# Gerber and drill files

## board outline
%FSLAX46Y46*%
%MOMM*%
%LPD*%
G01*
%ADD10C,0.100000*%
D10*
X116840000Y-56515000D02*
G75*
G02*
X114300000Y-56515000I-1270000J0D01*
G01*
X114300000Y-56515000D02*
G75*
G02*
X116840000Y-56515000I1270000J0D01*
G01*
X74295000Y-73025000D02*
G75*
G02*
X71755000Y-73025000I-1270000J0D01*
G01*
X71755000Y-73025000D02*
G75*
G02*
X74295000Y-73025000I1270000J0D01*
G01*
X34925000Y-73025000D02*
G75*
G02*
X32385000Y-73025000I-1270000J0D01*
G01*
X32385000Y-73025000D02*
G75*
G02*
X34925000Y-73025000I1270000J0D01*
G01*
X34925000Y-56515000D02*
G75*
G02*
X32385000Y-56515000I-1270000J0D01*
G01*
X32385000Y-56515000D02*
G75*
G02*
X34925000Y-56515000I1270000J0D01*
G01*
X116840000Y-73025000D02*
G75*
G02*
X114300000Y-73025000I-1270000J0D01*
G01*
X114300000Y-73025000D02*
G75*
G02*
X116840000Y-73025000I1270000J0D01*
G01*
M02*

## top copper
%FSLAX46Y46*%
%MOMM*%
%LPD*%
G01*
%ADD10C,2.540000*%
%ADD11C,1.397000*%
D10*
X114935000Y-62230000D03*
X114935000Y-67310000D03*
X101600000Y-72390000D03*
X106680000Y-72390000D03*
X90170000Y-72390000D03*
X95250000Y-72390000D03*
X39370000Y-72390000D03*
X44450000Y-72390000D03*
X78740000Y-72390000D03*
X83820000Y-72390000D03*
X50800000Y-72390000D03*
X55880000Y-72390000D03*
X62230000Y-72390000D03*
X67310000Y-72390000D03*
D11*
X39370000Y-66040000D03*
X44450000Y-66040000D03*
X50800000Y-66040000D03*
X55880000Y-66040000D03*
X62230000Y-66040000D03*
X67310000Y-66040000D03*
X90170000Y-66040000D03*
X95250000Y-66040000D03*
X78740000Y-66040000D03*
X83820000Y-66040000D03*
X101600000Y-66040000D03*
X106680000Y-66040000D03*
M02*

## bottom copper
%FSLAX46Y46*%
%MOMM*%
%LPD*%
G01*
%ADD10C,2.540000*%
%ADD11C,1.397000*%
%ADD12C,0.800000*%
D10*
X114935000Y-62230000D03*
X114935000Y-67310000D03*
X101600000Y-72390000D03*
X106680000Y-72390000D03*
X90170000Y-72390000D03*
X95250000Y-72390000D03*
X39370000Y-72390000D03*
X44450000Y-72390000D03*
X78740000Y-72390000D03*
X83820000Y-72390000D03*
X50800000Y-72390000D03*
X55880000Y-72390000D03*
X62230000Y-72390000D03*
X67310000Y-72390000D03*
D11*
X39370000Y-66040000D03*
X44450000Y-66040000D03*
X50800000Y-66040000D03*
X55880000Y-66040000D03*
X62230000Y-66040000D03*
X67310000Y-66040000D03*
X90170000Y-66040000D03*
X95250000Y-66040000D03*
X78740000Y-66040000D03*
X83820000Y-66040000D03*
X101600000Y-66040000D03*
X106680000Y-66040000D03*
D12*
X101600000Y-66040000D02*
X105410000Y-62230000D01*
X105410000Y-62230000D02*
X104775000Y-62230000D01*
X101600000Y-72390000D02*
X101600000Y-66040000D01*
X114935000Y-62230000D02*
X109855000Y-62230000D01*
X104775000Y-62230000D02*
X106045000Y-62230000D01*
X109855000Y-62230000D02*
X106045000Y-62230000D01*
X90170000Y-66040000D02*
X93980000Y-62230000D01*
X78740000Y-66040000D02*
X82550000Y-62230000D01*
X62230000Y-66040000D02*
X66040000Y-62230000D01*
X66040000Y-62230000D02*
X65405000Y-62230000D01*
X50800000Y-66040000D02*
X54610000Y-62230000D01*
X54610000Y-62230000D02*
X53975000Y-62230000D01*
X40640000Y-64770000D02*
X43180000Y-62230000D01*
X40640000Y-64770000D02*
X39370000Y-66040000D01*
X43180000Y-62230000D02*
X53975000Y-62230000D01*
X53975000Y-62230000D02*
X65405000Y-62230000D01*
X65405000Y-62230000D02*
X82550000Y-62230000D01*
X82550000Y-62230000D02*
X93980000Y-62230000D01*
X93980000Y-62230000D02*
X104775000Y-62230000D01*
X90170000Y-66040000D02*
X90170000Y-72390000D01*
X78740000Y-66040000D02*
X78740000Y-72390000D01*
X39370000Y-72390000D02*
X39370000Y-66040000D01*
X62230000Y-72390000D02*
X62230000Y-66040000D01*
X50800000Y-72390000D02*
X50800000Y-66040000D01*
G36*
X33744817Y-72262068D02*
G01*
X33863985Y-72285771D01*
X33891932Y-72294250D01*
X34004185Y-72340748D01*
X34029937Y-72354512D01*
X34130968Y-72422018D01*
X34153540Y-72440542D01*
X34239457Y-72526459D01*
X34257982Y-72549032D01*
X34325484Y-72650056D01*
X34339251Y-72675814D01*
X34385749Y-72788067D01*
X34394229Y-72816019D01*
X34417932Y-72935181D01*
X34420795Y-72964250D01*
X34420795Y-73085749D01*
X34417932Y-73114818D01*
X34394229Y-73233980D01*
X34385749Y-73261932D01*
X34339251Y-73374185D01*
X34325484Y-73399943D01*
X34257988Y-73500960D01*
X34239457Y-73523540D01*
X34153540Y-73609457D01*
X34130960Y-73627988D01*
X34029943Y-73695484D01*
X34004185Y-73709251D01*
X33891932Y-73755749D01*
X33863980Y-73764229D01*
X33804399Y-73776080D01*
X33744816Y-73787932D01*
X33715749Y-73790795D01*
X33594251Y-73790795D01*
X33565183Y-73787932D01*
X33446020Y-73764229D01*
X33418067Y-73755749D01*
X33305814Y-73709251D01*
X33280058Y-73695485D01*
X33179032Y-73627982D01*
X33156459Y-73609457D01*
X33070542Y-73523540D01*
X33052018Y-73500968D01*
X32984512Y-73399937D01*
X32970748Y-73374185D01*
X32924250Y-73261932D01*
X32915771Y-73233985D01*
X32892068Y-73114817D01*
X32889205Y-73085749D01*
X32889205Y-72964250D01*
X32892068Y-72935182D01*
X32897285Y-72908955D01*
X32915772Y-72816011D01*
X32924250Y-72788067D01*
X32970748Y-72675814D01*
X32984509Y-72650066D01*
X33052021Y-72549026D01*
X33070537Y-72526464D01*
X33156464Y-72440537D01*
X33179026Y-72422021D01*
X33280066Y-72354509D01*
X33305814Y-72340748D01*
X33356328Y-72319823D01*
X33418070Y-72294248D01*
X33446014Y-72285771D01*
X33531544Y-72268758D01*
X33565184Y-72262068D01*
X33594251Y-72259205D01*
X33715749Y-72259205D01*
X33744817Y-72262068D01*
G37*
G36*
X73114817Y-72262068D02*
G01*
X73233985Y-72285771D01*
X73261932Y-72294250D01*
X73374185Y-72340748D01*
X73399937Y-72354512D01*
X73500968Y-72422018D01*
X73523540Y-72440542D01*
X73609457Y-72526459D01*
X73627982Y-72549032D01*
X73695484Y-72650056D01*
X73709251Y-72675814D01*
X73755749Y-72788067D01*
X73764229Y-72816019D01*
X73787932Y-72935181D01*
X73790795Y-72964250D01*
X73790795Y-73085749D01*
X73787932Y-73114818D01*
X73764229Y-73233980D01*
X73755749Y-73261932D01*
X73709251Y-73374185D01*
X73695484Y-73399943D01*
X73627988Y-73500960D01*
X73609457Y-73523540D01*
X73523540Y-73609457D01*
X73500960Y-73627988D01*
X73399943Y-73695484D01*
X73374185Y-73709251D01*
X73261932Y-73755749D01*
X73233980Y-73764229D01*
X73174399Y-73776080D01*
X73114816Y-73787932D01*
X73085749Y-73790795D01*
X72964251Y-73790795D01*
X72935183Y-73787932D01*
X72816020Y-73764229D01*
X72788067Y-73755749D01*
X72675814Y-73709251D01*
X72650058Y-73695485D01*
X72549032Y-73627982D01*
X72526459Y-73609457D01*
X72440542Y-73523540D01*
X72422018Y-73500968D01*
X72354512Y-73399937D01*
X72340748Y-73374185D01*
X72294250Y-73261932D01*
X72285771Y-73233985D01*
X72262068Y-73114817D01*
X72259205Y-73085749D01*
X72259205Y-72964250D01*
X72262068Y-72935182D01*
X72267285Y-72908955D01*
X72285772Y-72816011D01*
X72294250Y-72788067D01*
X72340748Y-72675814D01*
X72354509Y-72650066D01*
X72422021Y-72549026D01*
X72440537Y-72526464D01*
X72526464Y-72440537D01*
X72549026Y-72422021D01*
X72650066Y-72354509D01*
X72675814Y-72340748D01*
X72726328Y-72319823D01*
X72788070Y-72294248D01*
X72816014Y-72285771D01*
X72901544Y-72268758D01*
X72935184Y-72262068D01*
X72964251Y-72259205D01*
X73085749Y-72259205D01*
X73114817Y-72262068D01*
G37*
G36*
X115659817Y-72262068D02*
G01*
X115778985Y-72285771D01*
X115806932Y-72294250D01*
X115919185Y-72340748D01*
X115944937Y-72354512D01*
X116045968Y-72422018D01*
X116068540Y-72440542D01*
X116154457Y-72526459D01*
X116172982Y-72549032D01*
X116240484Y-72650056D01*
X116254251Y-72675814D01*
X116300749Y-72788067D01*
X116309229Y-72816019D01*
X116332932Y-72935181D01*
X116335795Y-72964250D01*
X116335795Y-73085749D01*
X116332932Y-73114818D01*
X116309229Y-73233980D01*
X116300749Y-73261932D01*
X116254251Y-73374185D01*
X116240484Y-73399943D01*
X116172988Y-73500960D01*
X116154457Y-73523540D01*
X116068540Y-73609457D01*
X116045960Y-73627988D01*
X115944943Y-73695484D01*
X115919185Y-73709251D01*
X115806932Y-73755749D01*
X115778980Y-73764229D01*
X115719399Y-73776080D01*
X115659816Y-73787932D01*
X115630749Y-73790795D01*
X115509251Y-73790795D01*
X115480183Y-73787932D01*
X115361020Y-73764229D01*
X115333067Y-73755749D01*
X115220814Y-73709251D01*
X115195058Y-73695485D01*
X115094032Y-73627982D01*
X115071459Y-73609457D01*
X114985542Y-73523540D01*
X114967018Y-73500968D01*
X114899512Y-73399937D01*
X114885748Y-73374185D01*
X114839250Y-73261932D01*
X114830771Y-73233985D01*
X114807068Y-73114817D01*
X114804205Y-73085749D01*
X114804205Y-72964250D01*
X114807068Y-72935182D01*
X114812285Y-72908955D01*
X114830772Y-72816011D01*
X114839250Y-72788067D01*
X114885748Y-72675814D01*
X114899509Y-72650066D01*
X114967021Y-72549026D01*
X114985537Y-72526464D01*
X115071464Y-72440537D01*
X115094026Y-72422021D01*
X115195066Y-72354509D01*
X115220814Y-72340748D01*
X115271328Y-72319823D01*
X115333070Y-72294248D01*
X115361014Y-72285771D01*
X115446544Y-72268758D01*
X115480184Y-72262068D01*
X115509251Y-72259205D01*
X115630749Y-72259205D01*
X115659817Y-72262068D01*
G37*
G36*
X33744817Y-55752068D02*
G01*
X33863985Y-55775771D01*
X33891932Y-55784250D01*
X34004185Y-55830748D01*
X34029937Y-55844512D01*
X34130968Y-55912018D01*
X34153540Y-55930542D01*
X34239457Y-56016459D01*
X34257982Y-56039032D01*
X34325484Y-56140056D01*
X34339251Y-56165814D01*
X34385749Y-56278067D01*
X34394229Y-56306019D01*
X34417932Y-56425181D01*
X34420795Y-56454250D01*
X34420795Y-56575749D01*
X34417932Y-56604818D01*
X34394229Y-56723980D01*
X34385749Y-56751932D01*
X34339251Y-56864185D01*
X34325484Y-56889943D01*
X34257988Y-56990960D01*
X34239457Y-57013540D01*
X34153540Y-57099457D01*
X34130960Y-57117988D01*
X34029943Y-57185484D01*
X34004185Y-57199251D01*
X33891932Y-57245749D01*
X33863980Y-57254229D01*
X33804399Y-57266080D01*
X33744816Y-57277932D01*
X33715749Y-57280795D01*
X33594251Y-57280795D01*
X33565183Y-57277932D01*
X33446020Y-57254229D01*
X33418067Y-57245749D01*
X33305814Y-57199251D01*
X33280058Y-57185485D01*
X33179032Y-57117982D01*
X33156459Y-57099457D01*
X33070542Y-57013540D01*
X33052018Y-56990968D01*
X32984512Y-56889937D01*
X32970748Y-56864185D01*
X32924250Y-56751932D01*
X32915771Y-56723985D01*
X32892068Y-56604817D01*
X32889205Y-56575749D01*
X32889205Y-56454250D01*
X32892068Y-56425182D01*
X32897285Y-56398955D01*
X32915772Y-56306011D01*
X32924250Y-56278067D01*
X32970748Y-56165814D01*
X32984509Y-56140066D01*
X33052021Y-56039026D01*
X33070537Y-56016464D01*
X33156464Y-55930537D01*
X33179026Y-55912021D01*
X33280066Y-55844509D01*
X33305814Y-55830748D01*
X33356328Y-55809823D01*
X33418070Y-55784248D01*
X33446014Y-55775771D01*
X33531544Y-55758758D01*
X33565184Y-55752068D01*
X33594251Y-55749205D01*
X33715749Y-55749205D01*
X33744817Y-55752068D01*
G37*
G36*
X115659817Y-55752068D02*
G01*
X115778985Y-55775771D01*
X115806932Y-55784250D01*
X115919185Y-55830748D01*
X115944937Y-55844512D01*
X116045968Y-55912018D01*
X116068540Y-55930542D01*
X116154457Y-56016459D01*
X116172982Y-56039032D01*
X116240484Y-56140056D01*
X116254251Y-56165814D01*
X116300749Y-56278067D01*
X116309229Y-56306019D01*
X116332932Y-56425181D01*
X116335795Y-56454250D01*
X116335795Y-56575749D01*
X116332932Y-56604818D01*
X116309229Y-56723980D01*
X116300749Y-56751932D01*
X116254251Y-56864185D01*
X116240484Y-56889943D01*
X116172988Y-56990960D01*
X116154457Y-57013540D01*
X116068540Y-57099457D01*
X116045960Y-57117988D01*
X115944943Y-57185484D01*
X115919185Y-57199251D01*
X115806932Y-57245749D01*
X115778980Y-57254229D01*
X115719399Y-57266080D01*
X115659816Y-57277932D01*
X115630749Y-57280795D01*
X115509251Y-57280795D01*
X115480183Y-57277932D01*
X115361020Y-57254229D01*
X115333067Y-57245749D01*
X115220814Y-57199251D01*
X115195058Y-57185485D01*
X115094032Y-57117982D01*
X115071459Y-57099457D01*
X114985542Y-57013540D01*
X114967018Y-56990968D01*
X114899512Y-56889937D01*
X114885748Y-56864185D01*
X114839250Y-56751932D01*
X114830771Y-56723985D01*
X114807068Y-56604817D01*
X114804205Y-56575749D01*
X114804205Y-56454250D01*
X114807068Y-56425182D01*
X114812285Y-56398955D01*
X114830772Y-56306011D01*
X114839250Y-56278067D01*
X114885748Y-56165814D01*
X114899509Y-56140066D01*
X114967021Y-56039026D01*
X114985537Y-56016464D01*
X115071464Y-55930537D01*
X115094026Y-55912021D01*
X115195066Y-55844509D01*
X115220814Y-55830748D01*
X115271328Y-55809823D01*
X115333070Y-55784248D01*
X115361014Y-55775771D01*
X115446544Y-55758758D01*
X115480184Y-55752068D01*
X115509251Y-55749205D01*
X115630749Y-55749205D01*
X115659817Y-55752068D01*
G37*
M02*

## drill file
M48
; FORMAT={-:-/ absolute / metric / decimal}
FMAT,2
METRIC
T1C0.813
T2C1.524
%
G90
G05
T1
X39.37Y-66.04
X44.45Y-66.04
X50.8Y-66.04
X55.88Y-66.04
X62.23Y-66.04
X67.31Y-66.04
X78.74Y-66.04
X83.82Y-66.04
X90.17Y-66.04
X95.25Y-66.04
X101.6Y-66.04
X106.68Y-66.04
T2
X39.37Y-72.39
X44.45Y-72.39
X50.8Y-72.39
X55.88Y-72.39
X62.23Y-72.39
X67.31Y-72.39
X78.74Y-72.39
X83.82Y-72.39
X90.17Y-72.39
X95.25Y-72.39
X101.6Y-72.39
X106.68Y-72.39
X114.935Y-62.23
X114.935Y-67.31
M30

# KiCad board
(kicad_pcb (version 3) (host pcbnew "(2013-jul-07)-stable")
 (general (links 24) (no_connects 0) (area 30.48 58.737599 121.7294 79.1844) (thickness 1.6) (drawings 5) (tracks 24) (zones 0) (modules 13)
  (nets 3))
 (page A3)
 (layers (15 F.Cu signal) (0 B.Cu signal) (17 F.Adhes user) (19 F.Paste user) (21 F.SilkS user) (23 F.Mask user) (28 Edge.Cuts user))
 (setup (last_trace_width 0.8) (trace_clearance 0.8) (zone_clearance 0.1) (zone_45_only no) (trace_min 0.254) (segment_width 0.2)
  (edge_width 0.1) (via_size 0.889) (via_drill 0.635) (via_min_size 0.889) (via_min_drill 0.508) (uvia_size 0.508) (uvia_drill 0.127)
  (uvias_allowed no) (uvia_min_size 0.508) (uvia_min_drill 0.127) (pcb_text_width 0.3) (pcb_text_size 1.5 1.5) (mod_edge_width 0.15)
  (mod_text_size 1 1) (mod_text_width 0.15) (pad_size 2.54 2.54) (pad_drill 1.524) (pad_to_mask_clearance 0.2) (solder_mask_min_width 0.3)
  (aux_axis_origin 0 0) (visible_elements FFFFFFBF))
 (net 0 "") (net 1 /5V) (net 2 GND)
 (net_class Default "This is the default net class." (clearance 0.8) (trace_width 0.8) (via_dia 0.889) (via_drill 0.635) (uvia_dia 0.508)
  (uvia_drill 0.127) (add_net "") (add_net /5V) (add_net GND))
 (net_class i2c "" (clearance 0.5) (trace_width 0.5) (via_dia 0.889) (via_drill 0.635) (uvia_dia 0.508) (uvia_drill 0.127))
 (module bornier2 (layer F.Cu) (at 114.935 64.77 270)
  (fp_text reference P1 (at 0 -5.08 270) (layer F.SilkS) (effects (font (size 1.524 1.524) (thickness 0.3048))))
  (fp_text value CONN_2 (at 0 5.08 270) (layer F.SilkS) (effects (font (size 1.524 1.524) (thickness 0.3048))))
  (pad 1 thru_hole circle (at -2.54 0 270) (size 2.54 2.54) (drill 1.524) (layers *.Cu *.Mask F.SilkS) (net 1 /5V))
  (pad 2 thru_hole circle (at 2.54 0 270) (size 2.54 2.54) (drill 1.524) (layers *.Cu *.Mask F.SilkS) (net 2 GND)))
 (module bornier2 (layer F.Cu) (at 104.14 72.39)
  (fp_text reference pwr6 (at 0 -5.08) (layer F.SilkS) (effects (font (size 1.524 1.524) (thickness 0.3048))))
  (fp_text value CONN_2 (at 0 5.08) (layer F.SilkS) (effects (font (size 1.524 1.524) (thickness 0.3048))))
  (pad 1 thru_hole circle (at -2.54 0) (size 2.54 2.54) (drill 1.524) (layers *.Cu *.Mask F.SilkS) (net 1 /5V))
  (pad 2 thru_hole circle (at 2.54 0) (size 2.54 2.54) (drill 1.524) (layers *.Cu *.Mask F.SilkS) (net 2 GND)))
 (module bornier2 (layer F.Cu) (at 92.71 72.39)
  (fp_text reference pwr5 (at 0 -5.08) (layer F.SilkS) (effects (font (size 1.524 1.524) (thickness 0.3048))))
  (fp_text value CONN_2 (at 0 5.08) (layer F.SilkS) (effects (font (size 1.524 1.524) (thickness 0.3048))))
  (pad 1 thru_hole circle (at -2.54 0) (size 2.54 2.54) (drill 1.524) (layers *.Cu *.Mask F.SilkS) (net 1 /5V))
  (pad 2 thru_hole circle (at 2.54 0) (size 2.54 2.54) (drill 1.524) (layers *.Cu *.Mask F.SilkS) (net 2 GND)))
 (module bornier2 (layer F.Cu) (at 41.91 72.39)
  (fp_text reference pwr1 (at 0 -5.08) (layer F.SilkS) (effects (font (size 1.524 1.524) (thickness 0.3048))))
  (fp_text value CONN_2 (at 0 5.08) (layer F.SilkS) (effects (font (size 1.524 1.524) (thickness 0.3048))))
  (pad 1 thru_hole circle (at -2.54 0) (size 2.54 2.54) (drill 1.524) (layers *.Cu *.Mask F.SilkS) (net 1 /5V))
  (pad 2 thru_hole circle (at 2.54 0) (size 2.54 2.54) (drill 1.524) (layers *.Cu *.Mask F.SilkS) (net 2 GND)))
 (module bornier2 (layer F.Cu) (at 81.28 72.39)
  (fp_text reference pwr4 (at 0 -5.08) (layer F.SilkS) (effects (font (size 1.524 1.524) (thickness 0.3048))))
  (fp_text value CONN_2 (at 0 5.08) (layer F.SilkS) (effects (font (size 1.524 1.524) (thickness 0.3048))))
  (pad 1 thru_hole circle (at -2.54 0) (size 2.54 2.54) (drill 1.524) (layers *.Cu *.Mask F.SilkS) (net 1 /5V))
  (pad 2 thru_hole circle (at 2.54 0) (size 2.54 2.54) (drill 1.524) (layers *.Cu *.Mask F.SilkS) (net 2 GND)))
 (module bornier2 (layer F.Cu) (at 53.34 72.39)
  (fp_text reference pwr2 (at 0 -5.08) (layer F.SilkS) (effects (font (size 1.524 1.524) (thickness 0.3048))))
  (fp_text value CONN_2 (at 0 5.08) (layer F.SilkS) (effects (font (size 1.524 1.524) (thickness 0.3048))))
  (pad 1 thru_hole circle (at -2.54 0) (size 2.54 2.54) (drill 1.524) (layers *.Cu *.Mask F.SilkS) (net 1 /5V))
  (pad 2 thru_hole circle (at 2.54 0) (size 2.54 2.54) (drill 1.524) (layers *.Cu *.Mask F.SilkS) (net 2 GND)))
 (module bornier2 (layer F.Cu) (at 64.77 72.39)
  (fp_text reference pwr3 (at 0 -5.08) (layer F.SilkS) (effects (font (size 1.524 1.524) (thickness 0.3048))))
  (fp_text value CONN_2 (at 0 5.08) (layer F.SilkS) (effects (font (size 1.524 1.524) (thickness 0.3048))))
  (pad 1 thru_hole circle (at -2.54 0) (size 2.54 2.54) (drill 1.524) (layers *.Cu *.Mask F.SilkS) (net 1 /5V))
  (pad 2 thru_hole circle (at 2.54 0) (size 2.54 2.54) (drill 1.524) (layers *.Cu *.Mask F.SilkS) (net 2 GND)))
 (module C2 (layer F.Cu) (at 41.91 66.04)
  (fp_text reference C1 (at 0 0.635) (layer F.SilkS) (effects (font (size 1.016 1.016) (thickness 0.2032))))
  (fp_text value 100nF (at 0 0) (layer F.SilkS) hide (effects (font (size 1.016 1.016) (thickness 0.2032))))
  (pad 1 thru_hole circle (at -2.54 0) (size 1.397 1.397) (drill 0.8128) (layers *.Cu *.Mask F.SilkS) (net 1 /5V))
  (pad 2 thru_hole circle (at 2.54 0) (size 1.397 1.397) (drill 0.8128) (layers *.Cu *.Mask F.SilkS) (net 2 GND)))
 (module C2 (layer F.Cu) (at 53.34 66.04)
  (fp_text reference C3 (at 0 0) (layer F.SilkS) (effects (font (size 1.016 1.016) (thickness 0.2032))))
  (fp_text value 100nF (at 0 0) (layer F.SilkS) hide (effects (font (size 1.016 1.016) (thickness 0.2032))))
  (pad 1 thru_hole circle (at -2.54 0) (size 1.397 1.397) (drill 0.8128) (layers *.Cu *.Mask F.SilkS) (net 1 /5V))
  (pad 2 thru_hole circle (at 2.54 0) (size 1.397 1.397) (drill 0.8128) (layers *.Cu *.Mask F.SilkS) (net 2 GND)))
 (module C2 (layer F.Cu) (at 64.77 66.04)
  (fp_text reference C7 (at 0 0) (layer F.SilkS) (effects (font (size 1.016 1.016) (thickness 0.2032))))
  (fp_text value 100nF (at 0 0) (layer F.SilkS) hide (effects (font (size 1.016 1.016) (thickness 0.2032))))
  (pad 1 thru_hole circle (at -2.54 0) (size 1.397 1.397) (drill 0.8128) (layers *.Cu *.Mask F.SilkS) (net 1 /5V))
  (pad 2 thru_hole circle (at 2.54 0) (size 1.397 1.397) (drill 0.8128) (layers *.Cu *.Mask F.SilkS) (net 2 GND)))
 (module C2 (layer F.Cu) (at 92.71 66.04)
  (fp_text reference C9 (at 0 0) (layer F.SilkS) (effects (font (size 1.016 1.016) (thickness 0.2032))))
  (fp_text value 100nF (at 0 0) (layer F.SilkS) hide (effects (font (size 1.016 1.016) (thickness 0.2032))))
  (pad 1 thru_hole circle (at -2.54 0) (size 1.397 1.397) (drill 0.8128) (layers *.Cu *.Mask F.SilkS) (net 1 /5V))
  (pad 2 thru_hole circle (at 2.54 0) (size 1.397 1.397) (drill 0.8128) (layers *.Cu *.Mask F.SilkS) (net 2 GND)))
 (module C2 (layer F.Cu) (at 81.28 66.04)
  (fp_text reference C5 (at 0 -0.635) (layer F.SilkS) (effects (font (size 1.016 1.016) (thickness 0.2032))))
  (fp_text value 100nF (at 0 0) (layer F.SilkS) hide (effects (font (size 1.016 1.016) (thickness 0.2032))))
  (pad 1 thru_hole circle (at -2.54 0) (size 1.397 1.397) (drill 0.8128) (layers *.Cu *.Mask F.SilkS) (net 1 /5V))
  (pad 2 thru_hole circle (at 2.54 0) (size 1.397 1.397) (drill 0.8128) (layers *.Cu *.Mask F.SilkS) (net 2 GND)))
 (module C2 (layer F.Cu) (at 104.14 66.04)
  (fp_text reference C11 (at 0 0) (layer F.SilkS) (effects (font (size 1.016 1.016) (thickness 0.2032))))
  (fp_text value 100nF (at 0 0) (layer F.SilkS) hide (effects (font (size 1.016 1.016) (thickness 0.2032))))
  (pad 1 thru_hole circle (at -2.54 0) (size 1.397 1.397) (drill 0.8128) (layers *.Cu *.Mask F.SilkS) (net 1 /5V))
  (pad 2 thru_hole circle (at 2.54 0) (size 1.397 1.397) (drill 0.8128) (layers *.Cu *.Mask F.SilkS) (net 2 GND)))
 (gr_circle (center 115.57 56.515) (end 116.84 56.515) (layer Edge.Cuts) (width 0.1))
 (gr_circle (center 73.025 73.025) (end 74.295 73.025) (layer Edge.Cuts) (width 0.1))
 (gr_circle (center 33.655 73.025) (end 32.385 73.025) (layer Edge.Cuts) (width 0.1))
 (gr_circle (center 33.655 56.515) (end 34.925 56.515) (layer Edge.Cuts) (width 0.1))
 (gr_circle (center 115.57 73.025) (end 114.3 73.025) (layer Edge.Cuts) (width 0.1))
 (segment (start 101.6 66.04) (end 105.41 62.23) (width 0.8) (layer B.Cu) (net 1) (status 400000))
 (segment (start 105.41 62.23) (end 104.775 62.23) (width 0.8) (layer B.Cu) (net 1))
 (segment (start 101.6 72.39) (end 101.6 66.04) (width 0.8) (layer B.Cu) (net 1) (status C00000))
 (segment (start 114.935 62.23) (end 109.855 62.23) (width 0.8) (layer B.Cu) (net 1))
 (segment (start 104.775 62.23) (end 106.045 62.23) (width 0.8) (layer B.Cu) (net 1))
 (segment (start 109.855 62.23) (end 106.045 62.23) (width 0.8) (layer B.Cu) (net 1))
 (segment (start 90.17 66.04) (end 93.98 62.23) (width 0.8) (layer B.Cu) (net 1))
 (segment (start 78.74 66.04) (end 82.55 62.23) (width 0.8) (layer B.Cu) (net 1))
 (segment (start 62.23 66.04) (end 66.04 62.23) (width 0.8) (layer B.Cu) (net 1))
 (segment (start 66.04 62.23) (end 65.405 62.23) (width 0.8) (layer B.Cu) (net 1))
 (segment (start 50.8 66.04) (end 54.61 62.23) (width 0.8) (layer B.Cu) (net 1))
 (segment (start 54.61 62.23) (end 53.975 62.23) (width 0.8) (layer B.Cu) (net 1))
 (segment (start 40.64 64.77) (end 43.18 62.23) (width 0.8) (layer B.Cu) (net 1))
 (segment (start 40.64 64.77) (end 39.37 66.04) (width 0.8) (layer B.Cu) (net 1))
 (segment (start 43.18 62.23) (end 53.975 62.23) (width 0.8) (layer B.Cu) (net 1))
 (segment (start 53.975 62.23) (end 65.405 62.23) (width 0.8) (layer B.Cu) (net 1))
 (segment (start 65.405 62.23) (end 82.55 62.23) (width 0.8) (layer B.Cu) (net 1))
 (segment (start 82.55 62.23) (end 93.98 62.23) (width 0.8) (layer B.Cu) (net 1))
 (segment (start 93.98 62.23) (end 104.775 62.23) (width 0.8) (layer B.Cu) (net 1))
 (segment (start 90.17 66.04) (end 90.17 72.39) (width 0.8) (layer B.Cu) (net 1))
 (segment (start 78.74 66.04) (end 78.74 72.39) (width 0.8) (layer B.Cu) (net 1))
 (segment (start 39.37 72.39) (end 39.37 66.04) (width 0.8) (layer B.Cu) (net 1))
 (segment (start 62.23 72.39) (end 62.23 66.04) (width 0.8) (layer B.Cu) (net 1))
 (segment (start 50.8 72.39) (end 50.8 66.04) (width 0.8) (layer B.Cu) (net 1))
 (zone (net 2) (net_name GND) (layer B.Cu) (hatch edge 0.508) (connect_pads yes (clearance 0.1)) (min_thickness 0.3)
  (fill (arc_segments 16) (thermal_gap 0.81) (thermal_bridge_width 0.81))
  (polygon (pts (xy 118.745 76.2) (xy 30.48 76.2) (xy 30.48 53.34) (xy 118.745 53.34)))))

